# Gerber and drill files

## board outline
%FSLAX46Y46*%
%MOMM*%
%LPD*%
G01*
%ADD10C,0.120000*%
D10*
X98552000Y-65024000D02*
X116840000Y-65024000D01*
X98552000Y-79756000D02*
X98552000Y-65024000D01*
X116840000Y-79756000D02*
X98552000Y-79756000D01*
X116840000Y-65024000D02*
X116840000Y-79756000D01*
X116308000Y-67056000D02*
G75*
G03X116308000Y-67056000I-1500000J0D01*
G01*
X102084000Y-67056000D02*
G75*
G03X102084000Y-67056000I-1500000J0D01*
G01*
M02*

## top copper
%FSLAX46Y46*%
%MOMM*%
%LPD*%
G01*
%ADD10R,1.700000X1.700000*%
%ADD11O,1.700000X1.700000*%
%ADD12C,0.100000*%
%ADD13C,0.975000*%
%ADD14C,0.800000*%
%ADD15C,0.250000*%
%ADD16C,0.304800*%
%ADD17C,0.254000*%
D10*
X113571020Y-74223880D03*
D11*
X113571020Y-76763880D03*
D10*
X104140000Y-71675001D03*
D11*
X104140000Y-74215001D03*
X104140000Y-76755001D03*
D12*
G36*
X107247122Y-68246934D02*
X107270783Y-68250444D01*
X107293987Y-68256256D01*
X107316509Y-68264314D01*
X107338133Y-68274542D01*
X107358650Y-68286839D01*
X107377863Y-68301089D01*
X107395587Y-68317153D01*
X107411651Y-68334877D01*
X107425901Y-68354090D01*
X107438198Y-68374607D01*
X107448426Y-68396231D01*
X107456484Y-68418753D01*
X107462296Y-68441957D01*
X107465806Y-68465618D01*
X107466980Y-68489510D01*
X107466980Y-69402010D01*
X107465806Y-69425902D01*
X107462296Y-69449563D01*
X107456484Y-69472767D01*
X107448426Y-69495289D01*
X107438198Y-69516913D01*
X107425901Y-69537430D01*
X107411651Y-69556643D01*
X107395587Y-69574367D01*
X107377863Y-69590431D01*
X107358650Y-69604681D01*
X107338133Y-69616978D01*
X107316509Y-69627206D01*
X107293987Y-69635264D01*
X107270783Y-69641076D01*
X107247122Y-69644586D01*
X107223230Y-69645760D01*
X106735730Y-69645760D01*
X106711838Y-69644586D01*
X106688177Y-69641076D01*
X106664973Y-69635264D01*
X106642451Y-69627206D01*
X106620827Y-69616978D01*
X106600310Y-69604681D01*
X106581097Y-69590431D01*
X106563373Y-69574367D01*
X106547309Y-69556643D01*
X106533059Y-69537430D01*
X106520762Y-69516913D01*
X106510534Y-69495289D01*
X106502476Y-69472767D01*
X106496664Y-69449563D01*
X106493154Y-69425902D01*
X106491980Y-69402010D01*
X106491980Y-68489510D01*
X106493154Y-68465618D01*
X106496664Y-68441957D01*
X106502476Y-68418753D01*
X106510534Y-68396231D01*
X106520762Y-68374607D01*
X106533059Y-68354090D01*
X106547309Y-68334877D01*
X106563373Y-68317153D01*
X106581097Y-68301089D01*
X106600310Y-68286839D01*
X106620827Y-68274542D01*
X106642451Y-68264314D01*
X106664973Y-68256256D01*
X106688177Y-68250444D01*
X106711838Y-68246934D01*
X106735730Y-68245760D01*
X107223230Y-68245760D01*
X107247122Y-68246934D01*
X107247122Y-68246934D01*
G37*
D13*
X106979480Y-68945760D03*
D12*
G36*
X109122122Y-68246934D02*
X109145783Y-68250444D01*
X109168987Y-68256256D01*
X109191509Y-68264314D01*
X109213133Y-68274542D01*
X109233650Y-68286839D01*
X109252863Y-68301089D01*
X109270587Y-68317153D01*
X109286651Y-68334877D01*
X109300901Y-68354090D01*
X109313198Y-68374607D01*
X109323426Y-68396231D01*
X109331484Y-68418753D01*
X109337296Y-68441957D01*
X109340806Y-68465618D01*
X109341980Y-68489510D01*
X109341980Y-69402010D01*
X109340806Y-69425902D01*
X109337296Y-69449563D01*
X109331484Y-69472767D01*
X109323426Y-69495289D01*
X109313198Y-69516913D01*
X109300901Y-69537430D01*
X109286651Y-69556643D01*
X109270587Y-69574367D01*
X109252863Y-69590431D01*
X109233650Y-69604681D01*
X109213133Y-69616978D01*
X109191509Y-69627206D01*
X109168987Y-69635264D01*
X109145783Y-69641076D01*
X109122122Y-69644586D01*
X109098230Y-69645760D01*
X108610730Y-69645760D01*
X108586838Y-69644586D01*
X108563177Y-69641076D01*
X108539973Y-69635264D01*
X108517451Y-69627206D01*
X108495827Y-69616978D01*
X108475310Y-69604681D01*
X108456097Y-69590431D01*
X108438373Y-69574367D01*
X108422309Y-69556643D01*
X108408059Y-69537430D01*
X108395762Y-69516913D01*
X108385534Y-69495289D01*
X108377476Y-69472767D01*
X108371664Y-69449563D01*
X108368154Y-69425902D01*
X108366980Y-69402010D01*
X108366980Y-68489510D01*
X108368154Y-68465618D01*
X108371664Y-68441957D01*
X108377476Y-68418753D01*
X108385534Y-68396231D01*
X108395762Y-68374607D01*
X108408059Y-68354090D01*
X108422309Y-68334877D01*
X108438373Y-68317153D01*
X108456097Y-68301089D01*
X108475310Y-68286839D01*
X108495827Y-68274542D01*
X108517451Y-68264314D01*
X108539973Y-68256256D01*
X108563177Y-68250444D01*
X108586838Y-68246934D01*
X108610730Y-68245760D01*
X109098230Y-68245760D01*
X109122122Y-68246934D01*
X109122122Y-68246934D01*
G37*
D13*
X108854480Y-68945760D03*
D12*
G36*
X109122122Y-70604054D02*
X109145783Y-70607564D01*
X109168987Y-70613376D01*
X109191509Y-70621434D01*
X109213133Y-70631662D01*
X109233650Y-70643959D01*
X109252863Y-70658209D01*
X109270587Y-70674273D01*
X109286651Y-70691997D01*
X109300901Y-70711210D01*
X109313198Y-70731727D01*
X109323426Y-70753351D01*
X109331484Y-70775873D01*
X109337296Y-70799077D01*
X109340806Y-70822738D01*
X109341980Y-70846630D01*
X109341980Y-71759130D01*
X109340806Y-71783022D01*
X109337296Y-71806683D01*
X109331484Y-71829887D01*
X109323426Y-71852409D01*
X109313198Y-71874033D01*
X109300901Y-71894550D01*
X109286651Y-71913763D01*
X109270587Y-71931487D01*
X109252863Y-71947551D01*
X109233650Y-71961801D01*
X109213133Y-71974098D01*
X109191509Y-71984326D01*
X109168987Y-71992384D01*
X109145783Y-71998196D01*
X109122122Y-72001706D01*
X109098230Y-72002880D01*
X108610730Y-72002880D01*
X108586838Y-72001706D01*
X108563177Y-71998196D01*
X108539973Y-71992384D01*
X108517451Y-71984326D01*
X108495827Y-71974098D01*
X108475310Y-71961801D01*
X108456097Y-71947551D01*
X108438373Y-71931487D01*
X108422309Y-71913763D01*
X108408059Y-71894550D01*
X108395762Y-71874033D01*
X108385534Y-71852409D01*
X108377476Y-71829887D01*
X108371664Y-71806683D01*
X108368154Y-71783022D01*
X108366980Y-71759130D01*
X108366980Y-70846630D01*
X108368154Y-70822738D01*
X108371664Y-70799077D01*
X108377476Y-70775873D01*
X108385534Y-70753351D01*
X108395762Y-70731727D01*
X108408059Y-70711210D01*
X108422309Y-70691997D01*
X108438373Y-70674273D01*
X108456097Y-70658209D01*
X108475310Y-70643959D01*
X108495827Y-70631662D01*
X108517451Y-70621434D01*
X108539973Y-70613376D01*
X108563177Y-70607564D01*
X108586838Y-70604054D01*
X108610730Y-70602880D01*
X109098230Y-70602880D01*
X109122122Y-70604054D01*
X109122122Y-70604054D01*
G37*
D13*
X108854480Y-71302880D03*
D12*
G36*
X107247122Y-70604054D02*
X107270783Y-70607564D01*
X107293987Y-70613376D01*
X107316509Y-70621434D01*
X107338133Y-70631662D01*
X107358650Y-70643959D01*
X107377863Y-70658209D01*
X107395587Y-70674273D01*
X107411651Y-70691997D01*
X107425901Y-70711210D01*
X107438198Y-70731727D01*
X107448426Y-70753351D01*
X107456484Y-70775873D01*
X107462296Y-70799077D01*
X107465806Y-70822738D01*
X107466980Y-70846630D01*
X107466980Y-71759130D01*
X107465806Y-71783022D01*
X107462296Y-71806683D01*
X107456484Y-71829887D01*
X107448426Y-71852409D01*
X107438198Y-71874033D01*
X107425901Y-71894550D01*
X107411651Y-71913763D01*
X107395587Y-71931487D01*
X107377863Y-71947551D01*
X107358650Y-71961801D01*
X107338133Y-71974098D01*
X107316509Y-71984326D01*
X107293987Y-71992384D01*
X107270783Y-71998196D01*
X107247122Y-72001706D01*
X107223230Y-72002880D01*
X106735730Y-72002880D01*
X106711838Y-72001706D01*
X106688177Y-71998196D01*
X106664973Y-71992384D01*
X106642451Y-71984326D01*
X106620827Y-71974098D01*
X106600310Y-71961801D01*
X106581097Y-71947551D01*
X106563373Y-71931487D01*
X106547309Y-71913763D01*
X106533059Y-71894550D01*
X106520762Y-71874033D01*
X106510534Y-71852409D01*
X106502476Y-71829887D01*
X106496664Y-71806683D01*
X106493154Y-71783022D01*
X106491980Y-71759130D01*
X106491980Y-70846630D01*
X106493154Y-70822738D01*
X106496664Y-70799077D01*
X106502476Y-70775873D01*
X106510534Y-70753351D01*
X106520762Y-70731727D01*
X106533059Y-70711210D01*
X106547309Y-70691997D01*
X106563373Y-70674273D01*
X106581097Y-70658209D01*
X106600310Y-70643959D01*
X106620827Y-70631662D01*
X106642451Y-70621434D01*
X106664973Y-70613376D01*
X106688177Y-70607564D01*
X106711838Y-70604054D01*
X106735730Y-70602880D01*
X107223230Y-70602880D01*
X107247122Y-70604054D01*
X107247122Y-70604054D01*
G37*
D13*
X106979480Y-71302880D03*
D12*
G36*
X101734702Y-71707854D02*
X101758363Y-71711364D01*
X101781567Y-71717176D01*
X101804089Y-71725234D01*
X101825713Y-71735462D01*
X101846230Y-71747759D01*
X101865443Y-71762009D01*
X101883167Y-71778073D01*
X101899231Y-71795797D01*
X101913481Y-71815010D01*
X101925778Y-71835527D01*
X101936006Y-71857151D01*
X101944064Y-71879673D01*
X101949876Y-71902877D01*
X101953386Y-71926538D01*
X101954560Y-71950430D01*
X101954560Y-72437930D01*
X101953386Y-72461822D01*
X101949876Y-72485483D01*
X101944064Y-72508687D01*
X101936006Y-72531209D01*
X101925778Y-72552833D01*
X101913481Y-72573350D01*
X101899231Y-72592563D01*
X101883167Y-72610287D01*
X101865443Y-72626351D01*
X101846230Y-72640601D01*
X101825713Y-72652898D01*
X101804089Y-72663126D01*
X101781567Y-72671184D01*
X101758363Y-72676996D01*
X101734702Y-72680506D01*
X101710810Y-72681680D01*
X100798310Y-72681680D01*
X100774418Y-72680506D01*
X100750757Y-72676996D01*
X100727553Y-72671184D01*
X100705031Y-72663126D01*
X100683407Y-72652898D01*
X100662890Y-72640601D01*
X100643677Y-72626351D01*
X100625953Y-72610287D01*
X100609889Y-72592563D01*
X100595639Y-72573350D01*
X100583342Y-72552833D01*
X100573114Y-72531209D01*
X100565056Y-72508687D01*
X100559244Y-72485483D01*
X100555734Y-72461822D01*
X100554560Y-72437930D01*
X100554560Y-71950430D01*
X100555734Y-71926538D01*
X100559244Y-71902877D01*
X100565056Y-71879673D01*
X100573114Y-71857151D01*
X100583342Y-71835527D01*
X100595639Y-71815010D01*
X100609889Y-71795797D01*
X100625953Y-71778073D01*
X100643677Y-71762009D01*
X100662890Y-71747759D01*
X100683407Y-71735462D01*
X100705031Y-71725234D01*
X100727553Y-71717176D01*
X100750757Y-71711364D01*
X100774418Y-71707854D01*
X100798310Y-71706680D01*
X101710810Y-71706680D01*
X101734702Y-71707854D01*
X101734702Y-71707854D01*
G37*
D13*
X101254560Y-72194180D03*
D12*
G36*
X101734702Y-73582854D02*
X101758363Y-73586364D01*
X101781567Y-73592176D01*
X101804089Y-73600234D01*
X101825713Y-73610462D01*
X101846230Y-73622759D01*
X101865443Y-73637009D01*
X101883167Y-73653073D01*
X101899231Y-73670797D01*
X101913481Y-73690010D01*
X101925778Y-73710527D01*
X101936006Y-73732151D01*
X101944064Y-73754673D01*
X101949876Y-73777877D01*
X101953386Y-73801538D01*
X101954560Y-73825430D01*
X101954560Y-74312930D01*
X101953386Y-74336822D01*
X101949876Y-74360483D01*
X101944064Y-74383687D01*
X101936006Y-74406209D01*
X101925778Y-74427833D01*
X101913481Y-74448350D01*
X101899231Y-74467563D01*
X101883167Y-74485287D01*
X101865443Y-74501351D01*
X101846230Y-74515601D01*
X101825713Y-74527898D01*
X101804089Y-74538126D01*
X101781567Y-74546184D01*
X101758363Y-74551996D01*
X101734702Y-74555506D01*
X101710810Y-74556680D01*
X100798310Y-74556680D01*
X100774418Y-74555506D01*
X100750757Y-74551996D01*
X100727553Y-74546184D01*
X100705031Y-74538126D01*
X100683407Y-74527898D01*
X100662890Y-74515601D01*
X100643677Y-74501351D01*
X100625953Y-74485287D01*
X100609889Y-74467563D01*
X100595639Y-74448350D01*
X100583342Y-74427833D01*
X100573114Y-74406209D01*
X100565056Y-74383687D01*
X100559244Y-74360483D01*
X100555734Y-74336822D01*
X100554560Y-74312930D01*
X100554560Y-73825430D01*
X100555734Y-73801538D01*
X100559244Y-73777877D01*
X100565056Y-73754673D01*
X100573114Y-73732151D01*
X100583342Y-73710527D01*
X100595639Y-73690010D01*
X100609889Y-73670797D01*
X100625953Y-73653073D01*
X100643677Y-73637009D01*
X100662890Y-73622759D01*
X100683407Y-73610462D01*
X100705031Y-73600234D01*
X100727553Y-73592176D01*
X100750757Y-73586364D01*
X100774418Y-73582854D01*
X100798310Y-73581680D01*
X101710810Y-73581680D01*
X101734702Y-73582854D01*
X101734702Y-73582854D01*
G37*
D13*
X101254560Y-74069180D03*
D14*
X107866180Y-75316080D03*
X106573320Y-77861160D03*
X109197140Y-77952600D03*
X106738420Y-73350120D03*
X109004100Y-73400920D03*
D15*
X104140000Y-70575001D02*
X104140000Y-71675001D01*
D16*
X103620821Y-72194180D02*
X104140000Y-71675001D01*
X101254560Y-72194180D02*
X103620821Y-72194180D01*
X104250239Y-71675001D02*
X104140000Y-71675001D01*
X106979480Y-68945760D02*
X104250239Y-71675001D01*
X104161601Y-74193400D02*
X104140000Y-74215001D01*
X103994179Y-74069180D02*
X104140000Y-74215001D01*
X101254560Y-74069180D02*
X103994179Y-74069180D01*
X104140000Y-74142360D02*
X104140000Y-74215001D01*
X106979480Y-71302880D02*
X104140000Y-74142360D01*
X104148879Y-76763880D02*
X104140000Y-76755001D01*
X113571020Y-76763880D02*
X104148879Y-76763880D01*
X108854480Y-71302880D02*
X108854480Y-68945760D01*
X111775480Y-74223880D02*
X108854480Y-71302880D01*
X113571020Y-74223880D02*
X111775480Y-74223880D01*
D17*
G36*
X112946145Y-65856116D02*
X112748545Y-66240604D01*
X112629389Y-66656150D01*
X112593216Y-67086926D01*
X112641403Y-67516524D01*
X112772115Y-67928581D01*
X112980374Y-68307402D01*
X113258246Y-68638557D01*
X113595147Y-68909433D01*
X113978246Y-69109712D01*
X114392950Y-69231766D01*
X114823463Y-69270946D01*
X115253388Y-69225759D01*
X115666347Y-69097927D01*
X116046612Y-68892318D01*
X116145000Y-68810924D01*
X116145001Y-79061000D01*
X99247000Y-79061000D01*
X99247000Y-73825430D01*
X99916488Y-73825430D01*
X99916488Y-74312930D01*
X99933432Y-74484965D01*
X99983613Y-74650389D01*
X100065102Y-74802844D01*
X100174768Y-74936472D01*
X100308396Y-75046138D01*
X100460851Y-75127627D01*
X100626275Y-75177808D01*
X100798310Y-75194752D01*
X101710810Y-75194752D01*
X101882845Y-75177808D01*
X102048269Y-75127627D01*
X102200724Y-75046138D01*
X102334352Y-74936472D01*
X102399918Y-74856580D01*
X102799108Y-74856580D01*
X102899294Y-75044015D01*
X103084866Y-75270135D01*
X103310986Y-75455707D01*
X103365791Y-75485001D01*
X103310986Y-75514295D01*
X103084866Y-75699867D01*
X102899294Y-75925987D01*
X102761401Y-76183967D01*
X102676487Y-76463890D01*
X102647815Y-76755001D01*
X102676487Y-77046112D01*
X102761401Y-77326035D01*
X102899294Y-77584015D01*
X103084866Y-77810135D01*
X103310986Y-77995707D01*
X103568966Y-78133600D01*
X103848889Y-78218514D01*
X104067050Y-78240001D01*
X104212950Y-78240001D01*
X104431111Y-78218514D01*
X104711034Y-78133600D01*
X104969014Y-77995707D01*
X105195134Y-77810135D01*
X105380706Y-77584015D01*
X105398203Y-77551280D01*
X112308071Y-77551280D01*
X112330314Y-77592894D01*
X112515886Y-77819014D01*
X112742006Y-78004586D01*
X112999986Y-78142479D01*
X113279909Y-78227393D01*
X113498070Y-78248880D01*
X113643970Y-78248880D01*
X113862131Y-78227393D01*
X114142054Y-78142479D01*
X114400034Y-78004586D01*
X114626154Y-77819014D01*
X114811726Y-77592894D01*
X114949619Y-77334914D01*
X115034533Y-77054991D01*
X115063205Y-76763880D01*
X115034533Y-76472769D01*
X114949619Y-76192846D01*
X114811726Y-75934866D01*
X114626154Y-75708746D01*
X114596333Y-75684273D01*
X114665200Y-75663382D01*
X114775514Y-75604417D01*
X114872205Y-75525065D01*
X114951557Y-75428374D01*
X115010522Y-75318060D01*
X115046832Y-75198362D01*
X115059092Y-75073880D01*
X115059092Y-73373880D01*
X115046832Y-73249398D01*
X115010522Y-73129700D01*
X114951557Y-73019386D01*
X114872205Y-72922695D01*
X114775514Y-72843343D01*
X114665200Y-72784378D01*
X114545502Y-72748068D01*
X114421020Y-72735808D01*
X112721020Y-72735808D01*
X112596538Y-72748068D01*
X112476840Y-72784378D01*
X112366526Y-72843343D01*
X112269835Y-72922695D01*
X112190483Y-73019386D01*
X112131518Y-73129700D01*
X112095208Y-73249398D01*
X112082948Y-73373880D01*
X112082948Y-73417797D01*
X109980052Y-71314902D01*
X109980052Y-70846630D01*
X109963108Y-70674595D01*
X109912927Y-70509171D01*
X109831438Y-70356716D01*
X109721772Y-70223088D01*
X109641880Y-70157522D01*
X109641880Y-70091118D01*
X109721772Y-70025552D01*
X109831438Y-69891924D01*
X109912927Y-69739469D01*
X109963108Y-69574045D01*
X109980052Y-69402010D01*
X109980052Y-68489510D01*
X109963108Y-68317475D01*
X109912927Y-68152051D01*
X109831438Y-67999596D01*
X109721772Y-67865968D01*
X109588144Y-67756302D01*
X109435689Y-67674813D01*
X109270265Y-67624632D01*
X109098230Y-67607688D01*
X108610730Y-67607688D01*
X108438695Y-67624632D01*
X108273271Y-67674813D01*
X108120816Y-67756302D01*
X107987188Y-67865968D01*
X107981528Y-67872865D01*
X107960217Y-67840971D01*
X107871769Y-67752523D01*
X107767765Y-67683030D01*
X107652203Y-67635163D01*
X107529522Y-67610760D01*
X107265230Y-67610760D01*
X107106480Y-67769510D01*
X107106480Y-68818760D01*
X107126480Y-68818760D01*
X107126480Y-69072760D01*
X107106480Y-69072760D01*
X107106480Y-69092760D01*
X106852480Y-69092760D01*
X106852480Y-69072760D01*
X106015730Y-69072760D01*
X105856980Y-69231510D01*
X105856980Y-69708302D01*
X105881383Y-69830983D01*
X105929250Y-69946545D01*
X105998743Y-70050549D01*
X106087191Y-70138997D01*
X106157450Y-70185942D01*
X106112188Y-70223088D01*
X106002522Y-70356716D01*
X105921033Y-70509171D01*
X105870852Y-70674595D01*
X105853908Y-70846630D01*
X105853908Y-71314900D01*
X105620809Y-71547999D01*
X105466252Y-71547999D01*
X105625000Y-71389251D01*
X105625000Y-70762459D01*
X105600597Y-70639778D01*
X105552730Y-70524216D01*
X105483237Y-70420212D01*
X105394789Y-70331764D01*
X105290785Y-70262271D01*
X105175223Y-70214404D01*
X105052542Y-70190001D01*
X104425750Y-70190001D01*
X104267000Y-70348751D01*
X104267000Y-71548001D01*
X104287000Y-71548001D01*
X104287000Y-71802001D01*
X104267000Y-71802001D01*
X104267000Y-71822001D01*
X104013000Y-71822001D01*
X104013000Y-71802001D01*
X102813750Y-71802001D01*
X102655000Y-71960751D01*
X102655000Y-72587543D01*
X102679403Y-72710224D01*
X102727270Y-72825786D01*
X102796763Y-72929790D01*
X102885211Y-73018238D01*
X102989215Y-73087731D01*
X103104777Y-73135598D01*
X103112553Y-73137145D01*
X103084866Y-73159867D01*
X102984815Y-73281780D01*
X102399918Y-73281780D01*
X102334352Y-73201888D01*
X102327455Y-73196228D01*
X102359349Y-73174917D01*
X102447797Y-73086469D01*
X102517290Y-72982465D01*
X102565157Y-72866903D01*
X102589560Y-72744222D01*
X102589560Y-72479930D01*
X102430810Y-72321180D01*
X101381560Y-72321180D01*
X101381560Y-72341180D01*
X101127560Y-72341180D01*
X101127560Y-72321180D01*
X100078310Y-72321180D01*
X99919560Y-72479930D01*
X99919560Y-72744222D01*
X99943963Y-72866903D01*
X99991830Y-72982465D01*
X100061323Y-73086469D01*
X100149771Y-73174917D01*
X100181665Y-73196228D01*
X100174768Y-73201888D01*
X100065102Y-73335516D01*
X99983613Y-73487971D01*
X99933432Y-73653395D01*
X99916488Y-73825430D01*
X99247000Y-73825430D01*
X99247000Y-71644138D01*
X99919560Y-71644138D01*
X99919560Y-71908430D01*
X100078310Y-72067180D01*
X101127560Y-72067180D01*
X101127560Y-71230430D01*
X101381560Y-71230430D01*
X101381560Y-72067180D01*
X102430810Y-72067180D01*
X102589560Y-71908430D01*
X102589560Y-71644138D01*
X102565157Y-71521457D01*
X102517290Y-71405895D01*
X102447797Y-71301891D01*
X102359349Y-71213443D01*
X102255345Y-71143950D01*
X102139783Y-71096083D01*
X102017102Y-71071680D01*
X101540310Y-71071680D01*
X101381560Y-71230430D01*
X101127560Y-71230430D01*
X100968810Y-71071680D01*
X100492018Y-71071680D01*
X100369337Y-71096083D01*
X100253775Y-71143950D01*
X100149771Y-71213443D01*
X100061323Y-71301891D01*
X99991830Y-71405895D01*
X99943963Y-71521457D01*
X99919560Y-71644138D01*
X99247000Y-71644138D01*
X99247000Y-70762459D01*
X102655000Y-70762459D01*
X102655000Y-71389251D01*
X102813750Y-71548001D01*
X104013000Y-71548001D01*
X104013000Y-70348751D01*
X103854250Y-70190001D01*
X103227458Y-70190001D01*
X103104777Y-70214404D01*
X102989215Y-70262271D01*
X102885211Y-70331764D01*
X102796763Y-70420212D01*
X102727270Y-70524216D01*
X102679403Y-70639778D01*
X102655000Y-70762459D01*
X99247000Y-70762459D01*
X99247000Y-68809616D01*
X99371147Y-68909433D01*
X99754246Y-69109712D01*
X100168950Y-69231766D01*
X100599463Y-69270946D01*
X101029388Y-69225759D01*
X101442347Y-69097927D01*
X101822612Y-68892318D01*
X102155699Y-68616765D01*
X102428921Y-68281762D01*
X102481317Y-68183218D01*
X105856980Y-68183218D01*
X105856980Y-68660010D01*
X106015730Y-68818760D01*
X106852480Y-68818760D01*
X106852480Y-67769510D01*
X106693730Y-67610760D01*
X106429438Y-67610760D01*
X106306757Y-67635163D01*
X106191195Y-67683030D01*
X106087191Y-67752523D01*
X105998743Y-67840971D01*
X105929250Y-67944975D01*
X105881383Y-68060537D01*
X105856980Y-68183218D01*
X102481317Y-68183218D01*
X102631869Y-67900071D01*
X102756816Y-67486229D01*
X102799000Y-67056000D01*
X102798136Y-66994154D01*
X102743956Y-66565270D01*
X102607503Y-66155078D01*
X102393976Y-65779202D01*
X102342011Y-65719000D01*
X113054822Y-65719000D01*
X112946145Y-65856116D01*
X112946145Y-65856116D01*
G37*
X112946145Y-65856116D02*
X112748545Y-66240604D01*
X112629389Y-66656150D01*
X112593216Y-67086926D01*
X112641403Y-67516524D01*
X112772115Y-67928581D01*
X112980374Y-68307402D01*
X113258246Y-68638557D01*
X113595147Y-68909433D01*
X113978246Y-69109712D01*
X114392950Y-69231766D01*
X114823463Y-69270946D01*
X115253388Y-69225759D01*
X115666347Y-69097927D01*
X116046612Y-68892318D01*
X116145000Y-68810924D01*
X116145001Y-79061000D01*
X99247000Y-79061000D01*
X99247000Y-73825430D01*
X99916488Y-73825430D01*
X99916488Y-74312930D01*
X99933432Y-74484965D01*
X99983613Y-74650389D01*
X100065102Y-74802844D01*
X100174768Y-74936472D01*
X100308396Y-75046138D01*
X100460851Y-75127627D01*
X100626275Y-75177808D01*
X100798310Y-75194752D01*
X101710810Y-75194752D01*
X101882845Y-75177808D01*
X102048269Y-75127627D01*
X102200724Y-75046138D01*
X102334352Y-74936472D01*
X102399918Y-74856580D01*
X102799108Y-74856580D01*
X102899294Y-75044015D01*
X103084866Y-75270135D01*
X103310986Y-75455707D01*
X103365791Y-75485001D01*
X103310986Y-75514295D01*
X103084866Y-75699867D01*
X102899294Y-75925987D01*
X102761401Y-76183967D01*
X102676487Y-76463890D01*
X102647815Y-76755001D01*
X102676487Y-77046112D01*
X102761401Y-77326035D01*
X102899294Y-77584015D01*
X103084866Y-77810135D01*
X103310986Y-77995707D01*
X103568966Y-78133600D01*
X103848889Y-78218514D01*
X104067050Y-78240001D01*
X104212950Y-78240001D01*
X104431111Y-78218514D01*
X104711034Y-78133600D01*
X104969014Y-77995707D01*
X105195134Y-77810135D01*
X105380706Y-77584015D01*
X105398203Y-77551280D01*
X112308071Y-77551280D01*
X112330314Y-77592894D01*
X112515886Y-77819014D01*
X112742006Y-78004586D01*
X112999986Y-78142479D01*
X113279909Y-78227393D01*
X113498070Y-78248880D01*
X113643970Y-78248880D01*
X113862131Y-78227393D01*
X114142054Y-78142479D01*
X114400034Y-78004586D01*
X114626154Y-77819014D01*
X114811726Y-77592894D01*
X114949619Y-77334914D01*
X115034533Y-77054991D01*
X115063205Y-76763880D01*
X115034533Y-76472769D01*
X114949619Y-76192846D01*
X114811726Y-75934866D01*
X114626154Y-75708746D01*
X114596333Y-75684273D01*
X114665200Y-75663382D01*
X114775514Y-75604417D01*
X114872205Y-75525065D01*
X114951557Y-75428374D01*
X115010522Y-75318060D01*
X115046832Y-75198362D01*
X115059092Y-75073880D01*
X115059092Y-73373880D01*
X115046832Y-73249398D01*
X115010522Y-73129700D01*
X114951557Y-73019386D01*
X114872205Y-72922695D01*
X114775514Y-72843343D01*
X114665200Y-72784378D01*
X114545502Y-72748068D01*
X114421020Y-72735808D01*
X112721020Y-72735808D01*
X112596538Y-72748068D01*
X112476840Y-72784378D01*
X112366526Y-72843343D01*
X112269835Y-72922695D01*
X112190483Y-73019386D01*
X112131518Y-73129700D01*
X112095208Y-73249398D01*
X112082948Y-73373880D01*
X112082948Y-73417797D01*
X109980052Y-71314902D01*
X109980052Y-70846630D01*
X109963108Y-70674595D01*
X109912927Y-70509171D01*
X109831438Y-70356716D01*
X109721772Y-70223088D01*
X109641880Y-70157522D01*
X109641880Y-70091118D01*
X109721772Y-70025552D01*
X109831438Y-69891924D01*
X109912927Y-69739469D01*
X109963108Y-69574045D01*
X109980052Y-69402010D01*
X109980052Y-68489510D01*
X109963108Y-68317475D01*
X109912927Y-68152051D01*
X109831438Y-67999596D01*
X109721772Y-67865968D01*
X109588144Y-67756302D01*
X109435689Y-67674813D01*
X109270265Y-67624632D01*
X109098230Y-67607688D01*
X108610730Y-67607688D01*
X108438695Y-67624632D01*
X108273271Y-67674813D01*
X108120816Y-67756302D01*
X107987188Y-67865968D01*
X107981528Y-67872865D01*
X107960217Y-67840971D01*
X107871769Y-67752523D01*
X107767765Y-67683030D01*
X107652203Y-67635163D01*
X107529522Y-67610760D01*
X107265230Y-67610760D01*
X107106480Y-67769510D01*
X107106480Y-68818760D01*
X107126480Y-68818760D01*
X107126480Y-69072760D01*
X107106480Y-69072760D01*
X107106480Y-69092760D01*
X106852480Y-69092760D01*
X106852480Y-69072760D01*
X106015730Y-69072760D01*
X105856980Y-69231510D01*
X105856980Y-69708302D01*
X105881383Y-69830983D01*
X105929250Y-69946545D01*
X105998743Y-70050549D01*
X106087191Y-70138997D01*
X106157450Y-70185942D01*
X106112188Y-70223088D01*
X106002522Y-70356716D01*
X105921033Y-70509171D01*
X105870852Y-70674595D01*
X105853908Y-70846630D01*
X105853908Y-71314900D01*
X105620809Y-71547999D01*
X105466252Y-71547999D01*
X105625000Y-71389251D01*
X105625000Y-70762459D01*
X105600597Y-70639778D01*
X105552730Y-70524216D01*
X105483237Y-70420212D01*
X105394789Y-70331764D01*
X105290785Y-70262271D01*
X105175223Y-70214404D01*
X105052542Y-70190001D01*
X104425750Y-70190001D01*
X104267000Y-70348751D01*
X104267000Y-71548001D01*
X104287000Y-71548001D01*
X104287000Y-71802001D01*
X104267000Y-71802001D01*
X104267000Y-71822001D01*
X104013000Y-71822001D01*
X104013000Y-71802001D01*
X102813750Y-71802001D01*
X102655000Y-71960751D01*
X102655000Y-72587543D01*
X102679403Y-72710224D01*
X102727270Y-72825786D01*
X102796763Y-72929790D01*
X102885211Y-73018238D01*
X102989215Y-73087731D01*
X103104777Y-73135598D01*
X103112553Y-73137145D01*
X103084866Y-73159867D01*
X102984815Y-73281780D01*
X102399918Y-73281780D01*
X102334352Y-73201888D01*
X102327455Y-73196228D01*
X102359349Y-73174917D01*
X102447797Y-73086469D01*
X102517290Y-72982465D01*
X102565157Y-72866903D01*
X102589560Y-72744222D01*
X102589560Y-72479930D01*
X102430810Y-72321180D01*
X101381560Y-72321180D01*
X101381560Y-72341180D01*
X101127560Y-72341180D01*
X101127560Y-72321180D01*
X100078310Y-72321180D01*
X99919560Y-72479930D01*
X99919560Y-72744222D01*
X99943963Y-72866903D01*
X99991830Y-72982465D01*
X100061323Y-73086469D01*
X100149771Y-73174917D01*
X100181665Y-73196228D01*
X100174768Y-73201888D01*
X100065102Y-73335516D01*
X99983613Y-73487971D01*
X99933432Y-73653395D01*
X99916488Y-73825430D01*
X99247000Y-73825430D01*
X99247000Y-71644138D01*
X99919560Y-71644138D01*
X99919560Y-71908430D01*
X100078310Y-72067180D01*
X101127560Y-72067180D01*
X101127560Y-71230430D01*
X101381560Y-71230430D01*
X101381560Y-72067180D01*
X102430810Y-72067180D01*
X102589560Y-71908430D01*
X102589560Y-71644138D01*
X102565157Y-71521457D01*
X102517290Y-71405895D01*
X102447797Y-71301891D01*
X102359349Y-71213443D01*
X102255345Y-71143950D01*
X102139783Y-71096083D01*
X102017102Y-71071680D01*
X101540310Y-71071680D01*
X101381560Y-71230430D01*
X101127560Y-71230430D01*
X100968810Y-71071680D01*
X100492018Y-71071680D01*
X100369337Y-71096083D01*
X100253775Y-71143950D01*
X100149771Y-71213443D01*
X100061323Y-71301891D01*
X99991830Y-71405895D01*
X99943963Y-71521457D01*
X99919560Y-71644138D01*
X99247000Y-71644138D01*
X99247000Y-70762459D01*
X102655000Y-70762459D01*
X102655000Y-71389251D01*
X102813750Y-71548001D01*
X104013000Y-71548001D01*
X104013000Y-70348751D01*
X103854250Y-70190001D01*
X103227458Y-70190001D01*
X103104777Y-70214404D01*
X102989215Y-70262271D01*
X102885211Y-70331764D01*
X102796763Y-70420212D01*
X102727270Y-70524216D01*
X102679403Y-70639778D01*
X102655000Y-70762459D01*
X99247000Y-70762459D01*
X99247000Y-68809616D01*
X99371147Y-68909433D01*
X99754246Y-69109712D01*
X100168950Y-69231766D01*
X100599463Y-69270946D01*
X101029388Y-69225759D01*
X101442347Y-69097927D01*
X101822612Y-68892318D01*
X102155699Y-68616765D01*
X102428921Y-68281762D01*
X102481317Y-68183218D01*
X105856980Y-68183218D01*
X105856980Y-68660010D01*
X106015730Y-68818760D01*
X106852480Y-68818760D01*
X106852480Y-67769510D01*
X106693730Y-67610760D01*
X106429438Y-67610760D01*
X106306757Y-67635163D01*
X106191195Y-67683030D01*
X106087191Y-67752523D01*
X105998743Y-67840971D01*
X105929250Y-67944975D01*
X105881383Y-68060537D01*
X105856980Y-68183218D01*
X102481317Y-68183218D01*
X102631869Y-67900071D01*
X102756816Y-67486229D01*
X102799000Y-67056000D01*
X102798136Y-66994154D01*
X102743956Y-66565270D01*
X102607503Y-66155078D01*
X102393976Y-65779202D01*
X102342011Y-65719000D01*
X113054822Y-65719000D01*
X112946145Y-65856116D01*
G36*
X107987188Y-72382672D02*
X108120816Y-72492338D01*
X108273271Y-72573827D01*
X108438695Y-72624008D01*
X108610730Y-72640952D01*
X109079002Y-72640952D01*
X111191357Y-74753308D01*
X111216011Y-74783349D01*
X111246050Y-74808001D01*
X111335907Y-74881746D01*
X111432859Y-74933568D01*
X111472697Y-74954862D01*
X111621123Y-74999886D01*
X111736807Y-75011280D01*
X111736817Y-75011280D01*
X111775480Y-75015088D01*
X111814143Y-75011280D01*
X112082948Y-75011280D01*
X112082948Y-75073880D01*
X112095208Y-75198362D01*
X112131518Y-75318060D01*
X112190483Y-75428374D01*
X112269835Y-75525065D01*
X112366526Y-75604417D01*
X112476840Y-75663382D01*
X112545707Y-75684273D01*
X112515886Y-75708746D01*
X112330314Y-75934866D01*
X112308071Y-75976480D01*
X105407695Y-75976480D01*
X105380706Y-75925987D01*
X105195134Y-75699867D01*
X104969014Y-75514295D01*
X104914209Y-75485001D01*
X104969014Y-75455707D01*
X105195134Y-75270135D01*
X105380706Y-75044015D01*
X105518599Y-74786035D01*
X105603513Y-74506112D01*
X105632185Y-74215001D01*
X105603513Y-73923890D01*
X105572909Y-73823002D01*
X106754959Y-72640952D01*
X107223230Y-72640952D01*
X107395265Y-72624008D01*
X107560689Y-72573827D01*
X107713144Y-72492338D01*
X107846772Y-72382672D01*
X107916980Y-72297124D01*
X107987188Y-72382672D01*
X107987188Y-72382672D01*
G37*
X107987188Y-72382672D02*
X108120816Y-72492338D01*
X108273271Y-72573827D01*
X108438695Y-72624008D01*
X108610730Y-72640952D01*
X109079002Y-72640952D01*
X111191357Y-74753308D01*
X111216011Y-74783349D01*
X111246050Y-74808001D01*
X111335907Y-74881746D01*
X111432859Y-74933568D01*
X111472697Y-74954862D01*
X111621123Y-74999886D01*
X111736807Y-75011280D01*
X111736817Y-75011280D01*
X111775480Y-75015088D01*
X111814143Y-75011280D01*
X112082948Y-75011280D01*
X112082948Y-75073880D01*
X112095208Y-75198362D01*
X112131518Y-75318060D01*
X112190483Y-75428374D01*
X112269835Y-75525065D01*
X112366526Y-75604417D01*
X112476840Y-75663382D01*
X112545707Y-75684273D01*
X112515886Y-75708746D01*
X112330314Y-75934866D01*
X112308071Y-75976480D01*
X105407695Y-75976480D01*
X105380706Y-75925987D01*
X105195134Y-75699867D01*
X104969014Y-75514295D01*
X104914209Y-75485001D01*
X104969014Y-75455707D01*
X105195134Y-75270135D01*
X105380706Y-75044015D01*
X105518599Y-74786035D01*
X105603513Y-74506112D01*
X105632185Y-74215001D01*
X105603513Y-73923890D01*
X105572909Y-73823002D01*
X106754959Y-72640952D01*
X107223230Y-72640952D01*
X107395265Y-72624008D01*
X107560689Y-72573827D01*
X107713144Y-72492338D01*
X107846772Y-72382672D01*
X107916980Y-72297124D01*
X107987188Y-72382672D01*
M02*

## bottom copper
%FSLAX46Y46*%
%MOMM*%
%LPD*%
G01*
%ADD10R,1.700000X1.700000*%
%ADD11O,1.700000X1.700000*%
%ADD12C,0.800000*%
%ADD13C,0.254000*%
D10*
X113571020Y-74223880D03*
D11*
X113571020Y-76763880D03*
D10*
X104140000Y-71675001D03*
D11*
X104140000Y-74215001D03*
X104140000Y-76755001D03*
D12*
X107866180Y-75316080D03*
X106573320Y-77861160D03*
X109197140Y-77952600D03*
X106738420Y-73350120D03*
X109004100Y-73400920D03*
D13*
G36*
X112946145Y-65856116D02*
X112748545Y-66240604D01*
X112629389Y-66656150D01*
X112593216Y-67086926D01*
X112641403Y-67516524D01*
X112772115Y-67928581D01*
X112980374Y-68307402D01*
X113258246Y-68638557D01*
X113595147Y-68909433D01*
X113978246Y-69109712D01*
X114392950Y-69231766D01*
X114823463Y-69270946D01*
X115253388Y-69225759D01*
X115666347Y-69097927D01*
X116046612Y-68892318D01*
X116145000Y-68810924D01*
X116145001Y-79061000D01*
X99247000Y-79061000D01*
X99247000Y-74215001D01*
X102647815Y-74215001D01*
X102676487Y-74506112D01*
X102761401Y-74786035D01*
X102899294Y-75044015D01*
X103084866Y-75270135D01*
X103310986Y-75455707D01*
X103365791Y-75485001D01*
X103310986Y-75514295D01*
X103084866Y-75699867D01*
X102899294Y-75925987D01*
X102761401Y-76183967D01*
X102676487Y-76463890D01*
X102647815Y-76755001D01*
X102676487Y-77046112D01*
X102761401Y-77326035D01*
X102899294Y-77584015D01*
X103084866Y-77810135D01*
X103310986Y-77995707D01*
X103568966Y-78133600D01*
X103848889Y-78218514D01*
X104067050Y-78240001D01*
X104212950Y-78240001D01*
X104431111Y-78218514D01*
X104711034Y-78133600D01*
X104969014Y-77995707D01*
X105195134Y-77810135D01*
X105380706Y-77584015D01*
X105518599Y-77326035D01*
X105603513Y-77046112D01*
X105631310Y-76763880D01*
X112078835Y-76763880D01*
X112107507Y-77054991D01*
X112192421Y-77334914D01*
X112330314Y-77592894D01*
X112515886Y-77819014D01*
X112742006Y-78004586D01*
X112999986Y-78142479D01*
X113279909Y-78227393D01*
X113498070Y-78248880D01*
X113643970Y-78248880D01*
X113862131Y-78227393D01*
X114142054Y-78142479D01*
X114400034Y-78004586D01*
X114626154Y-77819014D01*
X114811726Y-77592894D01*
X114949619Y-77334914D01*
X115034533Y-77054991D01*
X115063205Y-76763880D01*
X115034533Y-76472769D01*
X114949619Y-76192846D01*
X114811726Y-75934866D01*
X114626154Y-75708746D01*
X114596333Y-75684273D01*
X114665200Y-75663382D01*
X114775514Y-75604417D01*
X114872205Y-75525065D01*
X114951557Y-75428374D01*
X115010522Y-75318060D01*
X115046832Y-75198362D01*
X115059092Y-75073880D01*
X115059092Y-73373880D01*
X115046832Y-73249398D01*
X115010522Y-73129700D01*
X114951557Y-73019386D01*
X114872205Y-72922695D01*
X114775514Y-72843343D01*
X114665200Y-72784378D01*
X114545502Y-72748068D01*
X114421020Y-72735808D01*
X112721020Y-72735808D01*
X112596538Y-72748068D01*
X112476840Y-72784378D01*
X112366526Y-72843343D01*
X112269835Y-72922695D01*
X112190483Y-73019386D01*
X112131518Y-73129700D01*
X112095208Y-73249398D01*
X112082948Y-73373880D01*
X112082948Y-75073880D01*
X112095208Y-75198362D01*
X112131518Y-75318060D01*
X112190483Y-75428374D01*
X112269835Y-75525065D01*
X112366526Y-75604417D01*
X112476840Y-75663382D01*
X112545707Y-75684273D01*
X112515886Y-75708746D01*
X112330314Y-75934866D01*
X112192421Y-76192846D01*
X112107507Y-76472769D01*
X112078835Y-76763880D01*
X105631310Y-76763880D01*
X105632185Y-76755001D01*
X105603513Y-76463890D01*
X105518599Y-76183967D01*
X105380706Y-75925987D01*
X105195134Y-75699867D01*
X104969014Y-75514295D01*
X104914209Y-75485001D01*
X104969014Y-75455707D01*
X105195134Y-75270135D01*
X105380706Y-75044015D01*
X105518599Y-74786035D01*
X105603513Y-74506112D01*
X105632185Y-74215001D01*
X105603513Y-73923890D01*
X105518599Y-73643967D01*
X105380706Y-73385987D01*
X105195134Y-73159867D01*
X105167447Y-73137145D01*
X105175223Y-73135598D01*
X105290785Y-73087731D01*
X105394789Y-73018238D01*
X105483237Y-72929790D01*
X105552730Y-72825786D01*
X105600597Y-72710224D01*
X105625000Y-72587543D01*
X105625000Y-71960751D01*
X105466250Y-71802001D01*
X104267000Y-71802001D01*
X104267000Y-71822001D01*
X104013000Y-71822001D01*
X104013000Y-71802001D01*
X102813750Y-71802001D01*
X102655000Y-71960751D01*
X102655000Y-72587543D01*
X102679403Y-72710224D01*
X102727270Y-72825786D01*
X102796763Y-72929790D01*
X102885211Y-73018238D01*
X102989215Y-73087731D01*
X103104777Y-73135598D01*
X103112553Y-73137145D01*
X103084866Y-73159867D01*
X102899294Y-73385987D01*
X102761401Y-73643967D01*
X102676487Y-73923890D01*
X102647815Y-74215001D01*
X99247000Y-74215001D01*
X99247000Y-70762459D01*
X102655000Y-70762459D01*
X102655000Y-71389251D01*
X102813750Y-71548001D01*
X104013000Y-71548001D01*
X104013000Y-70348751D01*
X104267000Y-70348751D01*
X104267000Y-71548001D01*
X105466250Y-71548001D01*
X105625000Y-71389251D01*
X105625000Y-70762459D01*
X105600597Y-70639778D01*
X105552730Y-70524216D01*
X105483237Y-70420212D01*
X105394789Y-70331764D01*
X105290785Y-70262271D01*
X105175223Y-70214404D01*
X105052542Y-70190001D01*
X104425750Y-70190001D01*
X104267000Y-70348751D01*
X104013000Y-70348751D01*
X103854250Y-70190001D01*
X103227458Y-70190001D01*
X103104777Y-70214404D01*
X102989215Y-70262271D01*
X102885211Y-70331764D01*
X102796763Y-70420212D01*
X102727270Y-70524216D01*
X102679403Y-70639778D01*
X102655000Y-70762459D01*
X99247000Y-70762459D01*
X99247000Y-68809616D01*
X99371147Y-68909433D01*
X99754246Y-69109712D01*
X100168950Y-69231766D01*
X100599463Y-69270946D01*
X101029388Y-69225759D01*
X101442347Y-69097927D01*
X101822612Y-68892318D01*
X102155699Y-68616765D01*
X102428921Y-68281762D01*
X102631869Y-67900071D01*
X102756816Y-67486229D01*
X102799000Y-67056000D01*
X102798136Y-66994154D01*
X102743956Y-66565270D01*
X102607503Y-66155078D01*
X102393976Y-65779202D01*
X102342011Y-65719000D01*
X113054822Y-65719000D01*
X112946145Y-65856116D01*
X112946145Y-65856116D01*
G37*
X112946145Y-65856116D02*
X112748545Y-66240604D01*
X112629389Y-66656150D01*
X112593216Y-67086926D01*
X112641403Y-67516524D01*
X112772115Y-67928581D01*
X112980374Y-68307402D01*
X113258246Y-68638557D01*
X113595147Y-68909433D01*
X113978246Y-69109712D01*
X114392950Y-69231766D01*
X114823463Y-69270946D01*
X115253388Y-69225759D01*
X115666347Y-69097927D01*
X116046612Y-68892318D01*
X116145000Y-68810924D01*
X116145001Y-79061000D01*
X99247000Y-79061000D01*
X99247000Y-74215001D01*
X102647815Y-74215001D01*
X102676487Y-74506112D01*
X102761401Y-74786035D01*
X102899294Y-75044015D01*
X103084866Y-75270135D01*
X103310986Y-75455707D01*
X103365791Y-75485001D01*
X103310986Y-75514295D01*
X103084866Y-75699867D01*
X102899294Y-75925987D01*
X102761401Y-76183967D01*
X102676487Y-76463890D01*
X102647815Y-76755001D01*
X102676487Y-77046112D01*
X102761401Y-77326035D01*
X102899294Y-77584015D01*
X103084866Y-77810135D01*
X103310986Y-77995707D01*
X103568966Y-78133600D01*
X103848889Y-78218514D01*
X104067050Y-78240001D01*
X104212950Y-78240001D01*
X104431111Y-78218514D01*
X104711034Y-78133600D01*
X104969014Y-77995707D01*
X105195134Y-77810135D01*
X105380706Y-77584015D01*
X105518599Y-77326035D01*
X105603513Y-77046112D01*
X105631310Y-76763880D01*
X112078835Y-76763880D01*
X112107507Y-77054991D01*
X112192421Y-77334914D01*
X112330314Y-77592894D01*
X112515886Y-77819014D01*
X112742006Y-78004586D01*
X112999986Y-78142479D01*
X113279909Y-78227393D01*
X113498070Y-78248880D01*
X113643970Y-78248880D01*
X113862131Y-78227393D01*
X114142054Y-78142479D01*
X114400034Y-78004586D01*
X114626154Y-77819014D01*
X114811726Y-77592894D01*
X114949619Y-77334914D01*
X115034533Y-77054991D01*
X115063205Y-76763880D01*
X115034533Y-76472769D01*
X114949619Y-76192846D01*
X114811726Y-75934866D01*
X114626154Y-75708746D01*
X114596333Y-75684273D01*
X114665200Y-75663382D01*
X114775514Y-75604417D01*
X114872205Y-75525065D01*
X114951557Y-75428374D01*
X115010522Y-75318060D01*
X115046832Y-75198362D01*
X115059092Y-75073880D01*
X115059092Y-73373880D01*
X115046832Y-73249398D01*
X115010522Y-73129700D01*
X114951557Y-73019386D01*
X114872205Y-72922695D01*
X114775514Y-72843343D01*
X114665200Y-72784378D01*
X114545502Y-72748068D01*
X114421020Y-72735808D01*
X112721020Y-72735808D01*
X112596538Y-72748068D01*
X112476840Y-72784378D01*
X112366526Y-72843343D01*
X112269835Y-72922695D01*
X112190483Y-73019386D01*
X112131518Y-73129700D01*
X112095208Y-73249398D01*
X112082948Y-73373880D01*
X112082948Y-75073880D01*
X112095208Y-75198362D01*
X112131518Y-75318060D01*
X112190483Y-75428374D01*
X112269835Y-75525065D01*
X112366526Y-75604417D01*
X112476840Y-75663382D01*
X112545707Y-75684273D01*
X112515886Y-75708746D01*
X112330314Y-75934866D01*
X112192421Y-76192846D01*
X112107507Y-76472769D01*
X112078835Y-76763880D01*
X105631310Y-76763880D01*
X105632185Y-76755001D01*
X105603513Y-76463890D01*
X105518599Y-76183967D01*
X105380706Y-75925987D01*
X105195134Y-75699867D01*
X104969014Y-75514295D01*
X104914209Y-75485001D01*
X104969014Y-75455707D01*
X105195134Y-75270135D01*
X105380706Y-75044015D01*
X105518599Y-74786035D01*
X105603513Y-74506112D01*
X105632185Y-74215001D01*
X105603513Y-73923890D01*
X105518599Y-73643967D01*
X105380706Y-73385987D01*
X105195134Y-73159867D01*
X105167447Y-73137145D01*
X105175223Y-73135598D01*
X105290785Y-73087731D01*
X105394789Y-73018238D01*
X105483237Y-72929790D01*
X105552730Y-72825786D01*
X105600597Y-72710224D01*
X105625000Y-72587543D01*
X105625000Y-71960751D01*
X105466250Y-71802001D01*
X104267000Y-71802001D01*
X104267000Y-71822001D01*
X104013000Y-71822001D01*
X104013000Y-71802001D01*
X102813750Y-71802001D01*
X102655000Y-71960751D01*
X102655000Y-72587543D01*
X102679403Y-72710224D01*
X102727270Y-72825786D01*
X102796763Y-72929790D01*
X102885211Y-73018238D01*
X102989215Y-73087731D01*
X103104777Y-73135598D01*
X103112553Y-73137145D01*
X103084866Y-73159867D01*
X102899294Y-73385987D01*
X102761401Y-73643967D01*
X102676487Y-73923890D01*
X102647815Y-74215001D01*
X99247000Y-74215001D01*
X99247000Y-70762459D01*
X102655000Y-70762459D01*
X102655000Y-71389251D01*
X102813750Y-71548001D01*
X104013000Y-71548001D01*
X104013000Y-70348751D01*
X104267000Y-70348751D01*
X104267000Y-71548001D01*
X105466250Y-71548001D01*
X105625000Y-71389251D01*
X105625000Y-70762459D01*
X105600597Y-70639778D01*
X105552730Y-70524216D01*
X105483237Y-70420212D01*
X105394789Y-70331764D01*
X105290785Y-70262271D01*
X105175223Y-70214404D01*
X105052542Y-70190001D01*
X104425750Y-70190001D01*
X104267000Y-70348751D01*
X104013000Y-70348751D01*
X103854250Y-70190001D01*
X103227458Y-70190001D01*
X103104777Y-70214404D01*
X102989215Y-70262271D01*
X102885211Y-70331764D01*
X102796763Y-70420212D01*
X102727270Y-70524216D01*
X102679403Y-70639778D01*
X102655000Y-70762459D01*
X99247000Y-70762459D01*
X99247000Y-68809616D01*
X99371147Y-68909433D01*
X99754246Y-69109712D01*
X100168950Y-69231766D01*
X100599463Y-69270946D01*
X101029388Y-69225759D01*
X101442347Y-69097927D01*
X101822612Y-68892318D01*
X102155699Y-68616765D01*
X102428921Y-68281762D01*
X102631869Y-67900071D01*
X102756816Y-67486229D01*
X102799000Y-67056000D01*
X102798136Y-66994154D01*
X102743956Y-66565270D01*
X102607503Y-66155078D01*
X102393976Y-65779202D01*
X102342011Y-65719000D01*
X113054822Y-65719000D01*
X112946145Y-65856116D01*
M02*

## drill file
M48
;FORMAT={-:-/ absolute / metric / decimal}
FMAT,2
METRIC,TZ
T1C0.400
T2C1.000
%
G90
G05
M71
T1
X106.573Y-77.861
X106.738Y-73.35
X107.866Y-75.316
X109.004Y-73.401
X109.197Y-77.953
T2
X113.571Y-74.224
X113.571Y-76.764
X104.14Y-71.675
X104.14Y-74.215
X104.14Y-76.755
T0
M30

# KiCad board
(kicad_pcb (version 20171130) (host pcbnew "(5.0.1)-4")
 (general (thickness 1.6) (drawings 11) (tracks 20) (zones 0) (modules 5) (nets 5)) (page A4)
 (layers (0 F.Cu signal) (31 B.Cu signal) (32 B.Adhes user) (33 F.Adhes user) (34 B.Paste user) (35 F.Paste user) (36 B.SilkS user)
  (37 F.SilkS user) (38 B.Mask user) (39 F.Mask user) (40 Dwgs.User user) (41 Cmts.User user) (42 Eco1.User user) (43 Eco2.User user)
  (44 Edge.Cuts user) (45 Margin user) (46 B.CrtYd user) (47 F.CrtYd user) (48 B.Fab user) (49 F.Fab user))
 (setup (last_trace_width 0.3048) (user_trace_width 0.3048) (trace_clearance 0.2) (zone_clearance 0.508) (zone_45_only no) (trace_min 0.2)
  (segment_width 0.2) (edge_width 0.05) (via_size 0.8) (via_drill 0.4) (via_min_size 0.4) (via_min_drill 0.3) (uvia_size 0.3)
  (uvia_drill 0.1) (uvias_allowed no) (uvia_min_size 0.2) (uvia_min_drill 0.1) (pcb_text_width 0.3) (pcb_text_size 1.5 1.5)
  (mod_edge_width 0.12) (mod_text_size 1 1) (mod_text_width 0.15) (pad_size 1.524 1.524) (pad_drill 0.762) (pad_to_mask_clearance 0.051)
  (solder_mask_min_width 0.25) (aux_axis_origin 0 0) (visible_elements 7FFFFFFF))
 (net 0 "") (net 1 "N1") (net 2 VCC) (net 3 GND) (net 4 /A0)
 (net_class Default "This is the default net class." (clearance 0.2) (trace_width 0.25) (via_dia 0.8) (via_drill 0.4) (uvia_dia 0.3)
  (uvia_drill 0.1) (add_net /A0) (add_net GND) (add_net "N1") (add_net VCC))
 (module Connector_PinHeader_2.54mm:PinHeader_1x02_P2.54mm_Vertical (layer F.Cu) (at 113.57102 74.22388)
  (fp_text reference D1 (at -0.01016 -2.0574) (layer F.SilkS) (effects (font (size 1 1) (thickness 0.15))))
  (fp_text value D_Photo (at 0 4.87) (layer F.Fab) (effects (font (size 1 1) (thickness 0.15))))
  (pad 1 thru_hole rect (at 0 0) (size 1.7 1.7) (drill 1) (layers *.Cu *.Mask) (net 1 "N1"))
  (pad 2 thru_hole oval (at 0 2.54) (size 1.7 1.7) (drill 1) (layers *.Cu *.Mask) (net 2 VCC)))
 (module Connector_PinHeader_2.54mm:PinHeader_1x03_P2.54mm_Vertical (layer F.Cu) (at 104.14 71.675001)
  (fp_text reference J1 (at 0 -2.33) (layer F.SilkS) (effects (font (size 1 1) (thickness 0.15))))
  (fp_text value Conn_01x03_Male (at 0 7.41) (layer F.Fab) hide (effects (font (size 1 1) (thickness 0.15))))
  (pad 1 thru_hole rect (at 0 0) (size 1.7 1.7) (drill 1) (layers *.Cu *.Mask) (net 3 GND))
  (pad 2 thru_hole oval (at 0 2.54) (size 1.7 1.7) (drill 1) (layers *.Cu *.Mask) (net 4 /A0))
  (pad 3 thru_hole oval (at 0 5.08) (size 1.7 1.7) (drill 1) (layers *.Cu *.Mask) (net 2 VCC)))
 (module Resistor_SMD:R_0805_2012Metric (layer F.Cu) (at 107.91698 68.94576)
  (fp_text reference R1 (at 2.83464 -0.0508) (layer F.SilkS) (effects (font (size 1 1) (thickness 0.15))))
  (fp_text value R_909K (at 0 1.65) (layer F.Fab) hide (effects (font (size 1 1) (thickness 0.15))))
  (pad 1 smd roundrect (at -0.9375 0) (size 0.975 1.4) (layers F.Cu F.Paste F.Mask) (roundrect_rratio 0.25) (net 3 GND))
  (pad 2 smd roundrect (at 0.9375 0) (size 0.975 1.4) (layers F.Cu F.Paste F.Mask) (roundrect_rratio 0.25) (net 1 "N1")))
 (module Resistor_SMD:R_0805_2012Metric (layer F.Cu) (at 107.91698 71.30288 180)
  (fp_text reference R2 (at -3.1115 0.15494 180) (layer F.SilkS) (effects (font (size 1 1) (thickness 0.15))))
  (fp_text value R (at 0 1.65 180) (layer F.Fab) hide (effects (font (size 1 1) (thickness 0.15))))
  (pad 1 smd roundrect (at -0.9375 0 180) (size 0.975 1.4) (layers F.Cu F.Paste F.Mask) (roundrect_rratio 0.25) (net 1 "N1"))
  (pad 2 smd roundrect (at 0.9375 0 180) (size 0.975 1.4) (layers F.Cu F.Paste F.Mask) (roundrect_rratio 0.25) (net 4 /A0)))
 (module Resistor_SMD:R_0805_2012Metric (layer F.Cu) (at 101.25456 73.13168 90)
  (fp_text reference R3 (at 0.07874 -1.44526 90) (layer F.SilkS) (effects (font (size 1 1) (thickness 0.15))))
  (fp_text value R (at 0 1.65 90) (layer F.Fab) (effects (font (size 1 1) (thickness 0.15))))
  (pad 2 smd roundrect (at 0.9375 0 90) (size 0.975 1.4) (layers F.Cu F.Paste F.Mask) (roundrect_rratio 0.25) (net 3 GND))
  (pad 1 smd roundrect (at -0.9375 0 90) (size 0.975 1.4) (layers F.Cu F.Paste F.Mask) (roundrect_rratio 0.25) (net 4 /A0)))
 (gr_line (start 98.552 65.024) (end 116.84 65.024) (layer Edge.Cuts) (width 0.12))
 (gr_line (start 98.552 79.756) (end 98.552 65.024) (layer Edge.Cuts) (width 0.12))
 (gr_line (start 116.84 79.756) (end 98.552 79.756) (layer Edge.Cuts) (width 0.12))
 (gr_line (start 116.84 65.024) (end 116.84 79.756) (layer Edge.Cuts) (width 0.12))
 (gr_circle (center 114.808 67.056) (end 116.308 67.056) (layer Edge.Cuts) (width 0.12))
 (gr_circle (center 100.584 67.056) (end 102.084 67.056) (layer Edge.Cuts) (width 0.12))
 (segment (start 104.14 70.575001) (end 104.14 71.675001) (width 0.25) (layer F.Cu) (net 3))
 (via (at 107.86618 75.31608) (size 0.8) (drill 0.4) (layers F.Cu B.Cu) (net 3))
 (via (at 106.57332 77.86116) (size 0.8) (drill 0.4) (layers F.Cu B.Cu) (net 3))
 (via (at 109.19714 77.9526) (size 0.8) (drill 0.4) (layers F.Cu B.Cu) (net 3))
 (via (at 106.73842 73.35012) (size 0.8) (drill 0.4) (layers F.Cu B.Cu) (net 3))
 (via (at 109.0041 73.40092) (size 0.8) (drill 0.4) (layers F.Cu B.Cu) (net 3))
 (segment (start 103.620821 72.19418) (end 104.14 71.675001) (width 0.3048) (layer F.Cu) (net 3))
 (segment (start 101.25456 72.19418) (end 103.620821 72.19418) (width 0.3048) (layer F.Cu) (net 3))
 (segment (start 104.250239 71.675001) (end 104.14 71.675001) (width 0.3048) (layer F.Cu) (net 3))
 (segment (start 106.97948 68.94576) (end 104.250239 71.675001) (width 0.3048) (layer F.Cu) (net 3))
 (segment (start 104.161601 74.1934) (end 104.14 74.215001) (width 0.3048) (layer F.Cu) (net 4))
 (segment (start 103.994179 74.06918) (end 104.14 74.215001) (width 0.3048) (layer F.Cu) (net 4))
 (segment (start 101.25456 74.06918) (end 103.994179 74.06918) (width 0.3048) (layer F.Cu) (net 4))
 (segment (start 104.14 74.14236) (end 104.14 74.215001) (width 0.3048) (layer F.Cu) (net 4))
 (segment (start 106.97948 71.30288) (end 104.14 74.14236) (width 0.3048) (layer F.Cu) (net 4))
 (segment (start 104.148879 76.76388) (end 104.14 76.755001) (width 0.3048) (layer F.Cu) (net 2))
 (segment (start 113.57102 76.76388) (end 104.148879 76.76388) (width 0.3048) (layer F.Cu) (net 2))
 (segment (start 108.85448 71.30288) (end 108.85448 68.94576) (width 0.3048) (layer F.Cu) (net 1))
 (segment (start 111.77548 74.22388) (end 108.85448 71.30288) (width 0.3048) (layer F.Cu) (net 1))
 (segment (start 113.57102 74.22388) (end 111.77548 74.22388) (width 0.3048) (layer F.Cu) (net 1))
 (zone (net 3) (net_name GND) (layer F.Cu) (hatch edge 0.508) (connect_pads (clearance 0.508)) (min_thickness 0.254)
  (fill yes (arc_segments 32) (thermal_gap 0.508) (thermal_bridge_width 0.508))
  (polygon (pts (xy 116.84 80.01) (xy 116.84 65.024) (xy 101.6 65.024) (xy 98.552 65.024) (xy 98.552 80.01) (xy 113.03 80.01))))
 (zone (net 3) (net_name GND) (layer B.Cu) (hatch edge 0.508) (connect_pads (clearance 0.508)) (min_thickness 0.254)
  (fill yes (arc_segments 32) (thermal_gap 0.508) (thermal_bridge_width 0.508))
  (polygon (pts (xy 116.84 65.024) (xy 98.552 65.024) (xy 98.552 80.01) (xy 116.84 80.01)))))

